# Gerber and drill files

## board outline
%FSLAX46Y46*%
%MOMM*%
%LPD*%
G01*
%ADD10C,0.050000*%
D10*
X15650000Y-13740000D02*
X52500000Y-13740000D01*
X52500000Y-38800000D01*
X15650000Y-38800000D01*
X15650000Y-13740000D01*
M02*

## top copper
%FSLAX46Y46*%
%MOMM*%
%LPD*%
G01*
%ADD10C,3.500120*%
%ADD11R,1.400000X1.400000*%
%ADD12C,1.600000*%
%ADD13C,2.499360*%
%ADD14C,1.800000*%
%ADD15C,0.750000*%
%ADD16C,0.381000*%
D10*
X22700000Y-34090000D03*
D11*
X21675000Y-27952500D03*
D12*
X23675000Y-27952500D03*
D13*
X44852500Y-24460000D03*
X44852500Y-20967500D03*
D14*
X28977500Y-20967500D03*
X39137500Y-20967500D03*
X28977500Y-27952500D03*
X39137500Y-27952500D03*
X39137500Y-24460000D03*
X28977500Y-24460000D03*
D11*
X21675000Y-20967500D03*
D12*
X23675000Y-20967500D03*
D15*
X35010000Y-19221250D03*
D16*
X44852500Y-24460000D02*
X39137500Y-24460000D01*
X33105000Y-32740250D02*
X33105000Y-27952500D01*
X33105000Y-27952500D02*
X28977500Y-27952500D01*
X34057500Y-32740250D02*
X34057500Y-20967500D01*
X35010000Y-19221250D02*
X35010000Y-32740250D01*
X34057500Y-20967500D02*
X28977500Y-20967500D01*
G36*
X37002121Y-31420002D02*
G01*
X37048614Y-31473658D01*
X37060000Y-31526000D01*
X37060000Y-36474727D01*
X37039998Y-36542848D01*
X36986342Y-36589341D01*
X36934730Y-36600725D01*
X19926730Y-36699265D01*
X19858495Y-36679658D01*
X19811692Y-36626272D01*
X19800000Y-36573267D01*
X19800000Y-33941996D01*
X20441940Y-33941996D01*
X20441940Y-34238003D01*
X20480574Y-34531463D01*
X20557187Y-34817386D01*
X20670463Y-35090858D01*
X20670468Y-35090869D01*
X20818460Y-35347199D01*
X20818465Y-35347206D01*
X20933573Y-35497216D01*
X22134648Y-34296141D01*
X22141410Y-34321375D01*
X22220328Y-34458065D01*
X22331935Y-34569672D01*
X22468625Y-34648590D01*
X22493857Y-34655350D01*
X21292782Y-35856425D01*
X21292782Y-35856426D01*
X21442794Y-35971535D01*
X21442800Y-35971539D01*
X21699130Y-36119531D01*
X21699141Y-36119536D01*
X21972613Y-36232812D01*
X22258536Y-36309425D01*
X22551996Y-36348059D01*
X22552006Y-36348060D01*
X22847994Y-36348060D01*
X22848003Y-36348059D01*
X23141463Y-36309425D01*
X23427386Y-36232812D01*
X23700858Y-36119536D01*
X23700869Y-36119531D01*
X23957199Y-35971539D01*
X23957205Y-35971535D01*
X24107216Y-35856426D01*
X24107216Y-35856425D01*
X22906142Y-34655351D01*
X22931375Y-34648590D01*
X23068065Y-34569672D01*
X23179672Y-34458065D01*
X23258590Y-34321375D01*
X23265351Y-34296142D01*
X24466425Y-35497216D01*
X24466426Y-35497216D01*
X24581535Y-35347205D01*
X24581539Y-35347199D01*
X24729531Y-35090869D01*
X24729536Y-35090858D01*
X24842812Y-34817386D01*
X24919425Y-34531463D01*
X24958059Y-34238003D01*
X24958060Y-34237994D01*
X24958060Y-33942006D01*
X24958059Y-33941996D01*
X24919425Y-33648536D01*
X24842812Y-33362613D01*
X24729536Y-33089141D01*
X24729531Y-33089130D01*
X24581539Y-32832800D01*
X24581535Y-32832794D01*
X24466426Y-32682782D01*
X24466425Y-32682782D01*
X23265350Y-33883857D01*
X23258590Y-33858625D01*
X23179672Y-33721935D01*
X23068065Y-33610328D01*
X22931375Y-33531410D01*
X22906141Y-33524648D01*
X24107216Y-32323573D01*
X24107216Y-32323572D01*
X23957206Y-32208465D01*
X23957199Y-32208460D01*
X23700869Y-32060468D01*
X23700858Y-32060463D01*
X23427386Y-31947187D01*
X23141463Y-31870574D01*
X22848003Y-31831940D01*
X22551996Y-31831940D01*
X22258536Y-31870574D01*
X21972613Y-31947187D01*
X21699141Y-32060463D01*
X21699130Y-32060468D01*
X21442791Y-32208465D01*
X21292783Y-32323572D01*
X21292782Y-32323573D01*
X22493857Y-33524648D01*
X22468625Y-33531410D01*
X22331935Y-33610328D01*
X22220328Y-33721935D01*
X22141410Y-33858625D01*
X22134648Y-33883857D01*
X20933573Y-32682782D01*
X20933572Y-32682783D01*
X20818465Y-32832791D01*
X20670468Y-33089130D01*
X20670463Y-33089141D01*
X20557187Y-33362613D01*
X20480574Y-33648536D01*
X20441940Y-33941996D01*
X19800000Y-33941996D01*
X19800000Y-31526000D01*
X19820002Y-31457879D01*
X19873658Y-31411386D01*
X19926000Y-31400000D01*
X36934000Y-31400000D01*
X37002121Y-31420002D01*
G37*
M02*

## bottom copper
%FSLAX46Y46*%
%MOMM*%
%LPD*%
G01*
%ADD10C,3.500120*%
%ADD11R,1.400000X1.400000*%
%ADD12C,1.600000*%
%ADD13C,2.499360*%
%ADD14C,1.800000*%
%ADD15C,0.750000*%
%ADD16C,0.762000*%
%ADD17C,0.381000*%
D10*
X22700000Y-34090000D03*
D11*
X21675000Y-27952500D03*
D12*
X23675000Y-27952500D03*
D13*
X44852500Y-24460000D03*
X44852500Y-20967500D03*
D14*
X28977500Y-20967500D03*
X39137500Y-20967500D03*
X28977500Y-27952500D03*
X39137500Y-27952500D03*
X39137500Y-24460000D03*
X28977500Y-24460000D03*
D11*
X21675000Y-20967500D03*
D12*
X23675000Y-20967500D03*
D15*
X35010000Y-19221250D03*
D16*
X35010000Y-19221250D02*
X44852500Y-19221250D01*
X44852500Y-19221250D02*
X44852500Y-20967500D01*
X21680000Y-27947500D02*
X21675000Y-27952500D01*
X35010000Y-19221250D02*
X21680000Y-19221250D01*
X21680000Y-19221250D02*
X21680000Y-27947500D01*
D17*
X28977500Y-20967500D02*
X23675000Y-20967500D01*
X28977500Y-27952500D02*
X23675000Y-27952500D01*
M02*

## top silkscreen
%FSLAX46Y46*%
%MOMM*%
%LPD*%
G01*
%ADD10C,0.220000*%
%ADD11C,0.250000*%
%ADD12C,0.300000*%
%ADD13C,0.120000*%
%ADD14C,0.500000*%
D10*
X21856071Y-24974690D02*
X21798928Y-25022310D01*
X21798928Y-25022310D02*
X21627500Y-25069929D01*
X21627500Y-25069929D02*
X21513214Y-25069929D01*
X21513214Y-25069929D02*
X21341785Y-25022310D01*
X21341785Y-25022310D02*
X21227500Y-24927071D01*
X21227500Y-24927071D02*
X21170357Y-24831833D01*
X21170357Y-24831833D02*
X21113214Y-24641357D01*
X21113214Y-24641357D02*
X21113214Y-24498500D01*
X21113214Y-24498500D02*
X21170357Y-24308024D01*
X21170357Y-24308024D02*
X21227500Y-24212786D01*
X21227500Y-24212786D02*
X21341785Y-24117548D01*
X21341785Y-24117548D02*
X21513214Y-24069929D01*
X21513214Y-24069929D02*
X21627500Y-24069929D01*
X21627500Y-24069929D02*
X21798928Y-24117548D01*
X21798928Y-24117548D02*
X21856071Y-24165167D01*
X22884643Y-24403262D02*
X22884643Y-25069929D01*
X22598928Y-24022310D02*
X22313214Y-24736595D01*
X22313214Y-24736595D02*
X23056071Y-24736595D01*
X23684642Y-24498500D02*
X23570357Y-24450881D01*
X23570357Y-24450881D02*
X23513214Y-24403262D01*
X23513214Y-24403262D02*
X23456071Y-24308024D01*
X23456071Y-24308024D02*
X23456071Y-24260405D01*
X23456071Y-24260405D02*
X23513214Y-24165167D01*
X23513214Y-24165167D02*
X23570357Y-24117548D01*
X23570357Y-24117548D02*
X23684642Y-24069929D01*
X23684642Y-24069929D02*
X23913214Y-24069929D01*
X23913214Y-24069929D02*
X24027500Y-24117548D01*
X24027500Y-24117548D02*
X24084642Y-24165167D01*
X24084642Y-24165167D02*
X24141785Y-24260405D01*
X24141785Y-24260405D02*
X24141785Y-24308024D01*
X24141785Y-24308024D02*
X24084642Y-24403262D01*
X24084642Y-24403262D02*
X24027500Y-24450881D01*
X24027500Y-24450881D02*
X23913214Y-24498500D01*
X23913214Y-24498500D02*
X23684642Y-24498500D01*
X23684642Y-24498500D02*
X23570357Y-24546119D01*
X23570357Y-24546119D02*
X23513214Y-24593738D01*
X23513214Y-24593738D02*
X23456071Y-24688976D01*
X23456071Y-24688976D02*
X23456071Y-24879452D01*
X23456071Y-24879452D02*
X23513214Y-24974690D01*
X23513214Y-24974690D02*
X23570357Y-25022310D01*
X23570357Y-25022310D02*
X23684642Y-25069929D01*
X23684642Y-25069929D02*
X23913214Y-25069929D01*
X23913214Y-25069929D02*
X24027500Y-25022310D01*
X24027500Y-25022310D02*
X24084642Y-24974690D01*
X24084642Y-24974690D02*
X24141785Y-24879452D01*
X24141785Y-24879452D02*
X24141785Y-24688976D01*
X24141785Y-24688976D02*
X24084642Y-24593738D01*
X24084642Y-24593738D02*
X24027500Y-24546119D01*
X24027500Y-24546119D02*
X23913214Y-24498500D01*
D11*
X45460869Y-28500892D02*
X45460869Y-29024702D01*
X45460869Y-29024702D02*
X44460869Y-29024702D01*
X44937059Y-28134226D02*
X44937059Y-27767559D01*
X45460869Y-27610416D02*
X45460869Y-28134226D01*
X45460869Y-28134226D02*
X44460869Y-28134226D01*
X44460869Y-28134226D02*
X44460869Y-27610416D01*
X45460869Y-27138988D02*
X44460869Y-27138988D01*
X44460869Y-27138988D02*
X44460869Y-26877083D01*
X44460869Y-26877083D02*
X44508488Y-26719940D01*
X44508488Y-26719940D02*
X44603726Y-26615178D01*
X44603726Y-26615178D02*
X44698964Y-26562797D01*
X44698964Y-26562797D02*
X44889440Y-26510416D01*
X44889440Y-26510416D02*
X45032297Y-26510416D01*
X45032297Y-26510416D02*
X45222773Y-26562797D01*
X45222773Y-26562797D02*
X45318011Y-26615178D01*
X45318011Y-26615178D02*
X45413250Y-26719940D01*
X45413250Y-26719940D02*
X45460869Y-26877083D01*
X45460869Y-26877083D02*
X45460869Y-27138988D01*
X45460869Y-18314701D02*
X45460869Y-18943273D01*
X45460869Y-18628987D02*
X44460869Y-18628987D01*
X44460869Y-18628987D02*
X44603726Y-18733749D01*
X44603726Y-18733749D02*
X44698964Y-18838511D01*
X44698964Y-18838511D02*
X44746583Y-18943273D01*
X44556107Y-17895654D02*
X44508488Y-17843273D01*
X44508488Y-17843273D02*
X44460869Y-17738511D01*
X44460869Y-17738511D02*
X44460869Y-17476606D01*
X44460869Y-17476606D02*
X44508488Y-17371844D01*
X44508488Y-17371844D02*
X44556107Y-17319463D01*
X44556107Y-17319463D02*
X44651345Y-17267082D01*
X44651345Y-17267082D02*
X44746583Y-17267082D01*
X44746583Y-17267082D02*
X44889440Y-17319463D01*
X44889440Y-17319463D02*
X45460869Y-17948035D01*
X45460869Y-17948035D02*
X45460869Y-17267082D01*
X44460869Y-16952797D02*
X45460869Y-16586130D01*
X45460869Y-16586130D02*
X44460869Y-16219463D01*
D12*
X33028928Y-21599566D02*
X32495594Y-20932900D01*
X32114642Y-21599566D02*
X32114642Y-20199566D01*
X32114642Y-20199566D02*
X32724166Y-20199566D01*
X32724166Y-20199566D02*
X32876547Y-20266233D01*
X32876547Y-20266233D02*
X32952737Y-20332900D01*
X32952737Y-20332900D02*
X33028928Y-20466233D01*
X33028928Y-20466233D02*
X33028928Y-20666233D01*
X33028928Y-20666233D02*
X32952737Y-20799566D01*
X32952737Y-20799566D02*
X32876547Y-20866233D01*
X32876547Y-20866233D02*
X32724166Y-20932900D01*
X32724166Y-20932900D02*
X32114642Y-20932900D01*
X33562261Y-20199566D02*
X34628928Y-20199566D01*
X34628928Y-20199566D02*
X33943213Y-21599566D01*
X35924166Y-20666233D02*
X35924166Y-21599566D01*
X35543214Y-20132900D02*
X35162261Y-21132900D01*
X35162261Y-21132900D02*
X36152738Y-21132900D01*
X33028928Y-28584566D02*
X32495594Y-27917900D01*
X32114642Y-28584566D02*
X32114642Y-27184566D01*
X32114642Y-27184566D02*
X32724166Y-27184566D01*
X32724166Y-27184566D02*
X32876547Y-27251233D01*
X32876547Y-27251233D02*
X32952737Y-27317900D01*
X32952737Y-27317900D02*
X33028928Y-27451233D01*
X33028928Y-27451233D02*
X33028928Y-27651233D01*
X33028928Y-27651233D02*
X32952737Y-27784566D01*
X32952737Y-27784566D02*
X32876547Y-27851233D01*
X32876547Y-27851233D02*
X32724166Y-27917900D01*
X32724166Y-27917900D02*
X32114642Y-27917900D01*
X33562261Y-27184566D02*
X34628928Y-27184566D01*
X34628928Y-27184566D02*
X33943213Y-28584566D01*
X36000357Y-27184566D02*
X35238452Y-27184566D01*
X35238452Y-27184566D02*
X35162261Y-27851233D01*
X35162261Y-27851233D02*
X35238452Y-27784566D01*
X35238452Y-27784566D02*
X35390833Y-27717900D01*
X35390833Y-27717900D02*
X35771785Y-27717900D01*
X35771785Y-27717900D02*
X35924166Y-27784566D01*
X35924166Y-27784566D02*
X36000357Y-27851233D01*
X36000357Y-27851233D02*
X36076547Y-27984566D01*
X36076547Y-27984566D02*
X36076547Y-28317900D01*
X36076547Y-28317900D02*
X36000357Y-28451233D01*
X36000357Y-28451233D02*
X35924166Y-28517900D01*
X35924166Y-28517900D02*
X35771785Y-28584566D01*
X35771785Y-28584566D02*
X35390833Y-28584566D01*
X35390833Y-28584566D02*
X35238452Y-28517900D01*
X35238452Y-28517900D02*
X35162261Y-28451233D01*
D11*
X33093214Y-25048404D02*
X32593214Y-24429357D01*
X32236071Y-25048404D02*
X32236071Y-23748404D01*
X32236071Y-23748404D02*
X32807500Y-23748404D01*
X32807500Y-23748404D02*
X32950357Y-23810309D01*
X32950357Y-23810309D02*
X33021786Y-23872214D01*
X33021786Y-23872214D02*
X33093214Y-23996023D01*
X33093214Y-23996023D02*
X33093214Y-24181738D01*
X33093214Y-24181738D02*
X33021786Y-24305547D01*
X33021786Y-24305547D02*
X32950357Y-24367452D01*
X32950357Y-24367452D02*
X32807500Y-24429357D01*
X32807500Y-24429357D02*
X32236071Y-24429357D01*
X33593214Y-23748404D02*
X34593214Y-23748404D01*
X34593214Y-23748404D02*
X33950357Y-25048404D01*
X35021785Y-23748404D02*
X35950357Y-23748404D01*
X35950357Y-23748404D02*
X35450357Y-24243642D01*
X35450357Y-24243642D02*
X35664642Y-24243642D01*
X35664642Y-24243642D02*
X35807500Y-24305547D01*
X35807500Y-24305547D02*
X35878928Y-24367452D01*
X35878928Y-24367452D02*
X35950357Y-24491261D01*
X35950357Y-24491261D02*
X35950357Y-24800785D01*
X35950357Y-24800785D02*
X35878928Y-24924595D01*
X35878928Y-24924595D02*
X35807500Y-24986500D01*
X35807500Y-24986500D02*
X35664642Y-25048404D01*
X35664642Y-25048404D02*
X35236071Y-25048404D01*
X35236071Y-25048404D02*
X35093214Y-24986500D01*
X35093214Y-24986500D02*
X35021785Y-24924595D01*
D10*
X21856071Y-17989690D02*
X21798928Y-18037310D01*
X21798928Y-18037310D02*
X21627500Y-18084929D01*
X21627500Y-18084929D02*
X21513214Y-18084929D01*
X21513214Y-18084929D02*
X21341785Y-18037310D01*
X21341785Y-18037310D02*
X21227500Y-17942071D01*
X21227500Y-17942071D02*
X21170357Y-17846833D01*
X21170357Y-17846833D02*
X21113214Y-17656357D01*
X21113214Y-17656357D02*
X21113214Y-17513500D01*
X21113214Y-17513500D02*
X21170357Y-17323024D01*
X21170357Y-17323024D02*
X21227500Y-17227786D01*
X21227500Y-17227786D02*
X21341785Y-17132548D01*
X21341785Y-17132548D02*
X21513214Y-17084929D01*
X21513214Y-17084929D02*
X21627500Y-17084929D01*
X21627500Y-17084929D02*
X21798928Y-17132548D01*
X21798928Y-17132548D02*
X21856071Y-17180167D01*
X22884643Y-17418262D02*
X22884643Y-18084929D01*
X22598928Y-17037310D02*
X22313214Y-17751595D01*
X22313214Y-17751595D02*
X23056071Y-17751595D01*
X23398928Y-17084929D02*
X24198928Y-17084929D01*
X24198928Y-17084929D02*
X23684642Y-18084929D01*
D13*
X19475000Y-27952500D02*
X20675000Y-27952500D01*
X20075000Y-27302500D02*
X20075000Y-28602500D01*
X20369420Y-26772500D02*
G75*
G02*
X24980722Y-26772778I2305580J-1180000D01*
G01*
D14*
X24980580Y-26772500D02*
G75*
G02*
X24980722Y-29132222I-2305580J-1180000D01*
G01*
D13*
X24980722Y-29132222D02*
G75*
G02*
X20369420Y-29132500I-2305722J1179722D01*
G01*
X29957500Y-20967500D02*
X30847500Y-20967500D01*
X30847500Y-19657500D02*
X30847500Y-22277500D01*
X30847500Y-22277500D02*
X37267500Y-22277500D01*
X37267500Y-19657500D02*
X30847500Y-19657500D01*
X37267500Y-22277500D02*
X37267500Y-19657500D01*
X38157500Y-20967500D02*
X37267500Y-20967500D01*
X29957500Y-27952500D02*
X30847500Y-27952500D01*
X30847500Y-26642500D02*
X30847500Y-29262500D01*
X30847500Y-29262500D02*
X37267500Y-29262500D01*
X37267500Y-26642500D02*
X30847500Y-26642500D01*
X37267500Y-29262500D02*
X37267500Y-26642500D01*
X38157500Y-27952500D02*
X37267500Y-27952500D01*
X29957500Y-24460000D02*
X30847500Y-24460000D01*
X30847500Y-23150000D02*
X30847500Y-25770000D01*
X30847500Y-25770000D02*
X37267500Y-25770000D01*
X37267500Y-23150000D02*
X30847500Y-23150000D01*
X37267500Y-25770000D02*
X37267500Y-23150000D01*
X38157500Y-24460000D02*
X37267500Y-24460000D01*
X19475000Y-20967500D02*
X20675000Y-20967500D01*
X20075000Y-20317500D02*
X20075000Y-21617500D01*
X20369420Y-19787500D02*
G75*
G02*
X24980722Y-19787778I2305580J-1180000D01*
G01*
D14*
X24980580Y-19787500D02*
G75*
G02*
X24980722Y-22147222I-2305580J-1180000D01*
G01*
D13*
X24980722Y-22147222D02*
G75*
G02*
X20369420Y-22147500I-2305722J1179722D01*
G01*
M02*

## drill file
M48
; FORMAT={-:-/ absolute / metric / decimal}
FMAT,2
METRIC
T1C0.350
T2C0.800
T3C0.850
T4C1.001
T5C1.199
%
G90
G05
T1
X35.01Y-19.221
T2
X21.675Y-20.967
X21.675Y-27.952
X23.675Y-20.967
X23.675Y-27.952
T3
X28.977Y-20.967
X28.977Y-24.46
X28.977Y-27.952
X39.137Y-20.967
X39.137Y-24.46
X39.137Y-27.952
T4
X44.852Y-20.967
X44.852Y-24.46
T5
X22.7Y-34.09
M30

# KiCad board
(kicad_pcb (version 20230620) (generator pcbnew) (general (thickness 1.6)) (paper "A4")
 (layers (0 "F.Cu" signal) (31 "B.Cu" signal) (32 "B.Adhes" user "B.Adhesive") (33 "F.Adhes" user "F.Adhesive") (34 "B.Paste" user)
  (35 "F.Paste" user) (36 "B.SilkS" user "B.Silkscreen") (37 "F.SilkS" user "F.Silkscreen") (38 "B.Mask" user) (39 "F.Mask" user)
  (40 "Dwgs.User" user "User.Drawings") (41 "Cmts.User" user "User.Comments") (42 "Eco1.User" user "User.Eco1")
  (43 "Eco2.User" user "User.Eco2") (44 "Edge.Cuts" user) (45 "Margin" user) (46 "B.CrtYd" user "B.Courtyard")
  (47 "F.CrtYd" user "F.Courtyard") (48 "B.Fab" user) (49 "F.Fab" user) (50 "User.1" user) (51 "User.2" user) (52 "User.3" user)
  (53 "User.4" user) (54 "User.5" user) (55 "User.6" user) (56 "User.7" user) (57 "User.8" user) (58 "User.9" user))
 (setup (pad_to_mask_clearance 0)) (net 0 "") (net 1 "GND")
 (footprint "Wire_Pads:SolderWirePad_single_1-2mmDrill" (layer "F.Cu") (at 22.7 34.09)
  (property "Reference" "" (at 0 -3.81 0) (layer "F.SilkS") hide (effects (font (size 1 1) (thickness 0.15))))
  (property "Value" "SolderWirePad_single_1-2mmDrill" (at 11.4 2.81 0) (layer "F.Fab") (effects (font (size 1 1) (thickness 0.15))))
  (pad "1" thru_hole circle (at 0 0) (size 3.50012 3.50012) (drill 1.19888) (layers "*.Cu" "*.Mask") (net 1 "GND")))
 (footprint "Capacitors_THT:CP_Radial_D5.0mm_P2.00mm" (layer "F.Cu") (at 21.675 27.9525)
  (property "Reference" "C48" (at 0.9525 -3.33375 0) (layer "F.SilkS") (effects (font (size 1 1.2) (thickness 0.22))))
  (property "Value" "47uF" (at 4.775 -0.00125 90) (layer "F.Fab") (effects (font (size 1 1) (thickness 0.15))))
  (fp_line (start -2.2 0) (end -1 0) (stroke (width 0.12) (type solid)) (layer "F.SilkS"))
  (fp_line (start -1.6 -0.65) (end -1.6 0.65) (stroke (width 0.12) (type solid)) (layer "F.SilkS"))
  (fp_arc (start -1.30558 -1.18) (mid 1.000156 -2.59) (end 3.305722 -1.179722) (stroke (width 0.12) (type solid)) (layer "F.SilkS"))
  (fp_arc (start 3.30558 -1.18) (mid 3.59 -0.000156) (end 3.305722 1.179722) (stroke (width 0.5) (type solid)) (layer "F.SilkS"))
  (fp_arc (start 3.305722 1.179722) (mid 1.000156 2.59) (end -1.30558 1.18) (stroke (width 0.12) (type solid)) (layer "F.SilkS"))
  (pad "1" thru_hole rect (at 0 0) (size 1.4 1.4) (drill 0.8) (layers "*.Cu" "*.Mask") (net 1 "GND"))
  (pad "2" thru_hole circle (at 2 0) (size 1.6 1.6) (drill 0.8) (layers "*.Cu" "*.Mask") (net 1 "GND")))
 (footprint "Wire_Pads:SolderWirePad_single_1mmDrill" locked (layer "F.Cu") (at 44.8525 24.46)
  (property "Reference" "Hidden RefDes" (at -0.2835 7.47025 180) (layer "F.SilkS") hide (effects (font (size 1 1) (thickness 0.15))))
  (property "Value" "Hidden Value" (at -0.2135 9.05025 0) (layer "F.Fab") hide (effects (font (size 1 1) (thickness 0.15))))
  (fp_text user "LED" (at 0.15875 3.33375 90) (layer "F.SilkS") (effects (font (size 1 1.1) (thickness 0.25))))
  (pad "1" thru_hole circle locked (at 0 0) (size 2.49936 2.49936) (drill 1.00076) (layers "*.Cu" "*.Mask")))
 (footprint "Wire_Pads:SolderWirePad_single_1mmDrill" (layer "F.Cu") (at 44.8525 20.9675)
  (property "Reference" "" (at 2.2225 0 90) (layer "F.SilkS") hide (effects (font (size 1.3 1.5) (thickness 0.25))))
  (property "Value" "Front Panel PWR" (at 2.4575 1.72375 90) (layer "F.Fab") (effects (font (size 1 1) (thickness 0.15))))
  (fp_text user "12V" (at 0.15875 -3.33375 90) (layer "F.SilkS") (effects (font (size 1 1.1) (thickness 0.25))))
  (pad "1" thru_hole circle (at 0 0) (size 2.49936 2.49936) (drill 1.00076) (layers "*.Cu" "*.Mask") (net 1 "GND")))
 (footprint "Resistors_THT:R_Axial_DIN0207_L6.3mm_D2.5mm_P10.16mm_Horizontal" (layer "F.Cu") (at 28.9775 20.9675)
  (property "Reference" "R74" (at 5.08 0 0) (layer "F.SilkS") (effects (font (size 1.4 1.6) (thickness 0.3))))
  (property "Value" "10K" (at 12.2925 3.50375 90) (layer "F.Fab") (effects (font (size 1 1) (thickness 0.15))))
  (fp_line (start 0.98 0) (end 1.87 0) (stroke (width 0.12) (type solid)) (layer "F.SilkS"))
  (fp_line (start 1.87 -1.31) (end 1.87 1.31) (stroke (width 0.12) (type solid)) (layer "F.SilkS"))
  (fp_line (start 1.87 1.31) (end 8.29 1.31) (stroke (width 0.12) (type solid)) (layer "F.SilkS"))
  (fp_line (start 8.29 -1.31) (end 1.87 -1.31) (stroke (width 0.12) (type solid)) (layer "F.SilkS"))
  (fp_line (start 8.29 1.31) (end 8.29 -1.31) (stroke (width 0.12) (type solid)) (layer "F.SilkS"))
  (fp_line (start 9.18 0) (end 8.29 0) (stroke (width 0.12) (type solid)) (layer "F.SilkS"))
  (pad "1" thru_hole circle (at 0 0) (size 1.8 1.8) (drill 0.85) (layers "*.Cu" "*.Mask") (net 1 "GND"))
  (pad "2" thru_hole circle (at 10.16 0) (size 1.8 1.8) (drill 0.85) (layers "*.Cu" "*.Mask")))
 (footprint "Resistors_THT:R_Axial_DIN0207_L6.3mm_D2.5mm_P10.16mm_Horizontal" (layer "F.Cu") (at 28.9775 27.9525)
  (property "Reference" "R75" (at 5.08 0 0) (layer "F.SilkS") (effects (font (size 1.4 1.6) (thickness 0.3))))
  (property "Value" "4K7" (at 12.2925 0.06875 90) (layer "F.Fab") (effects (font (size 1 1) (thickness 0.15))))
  (fp_line (start 0.98 0) (end 1.87 0) (stroke (width 0.12) (type solid)) (layer "F.SilkS"))
  (fp_line (start 1.87 -1.31) (end 1.87 1.31) (stroke (width 0.12) (type solid)) (layer "F.SilkS"))
  (fp_line (start 1.87 1.31) (end 8.29 1.31) (stroke (width 0.12) (type solid)) (layer "F.SilkS"))
  (fp_line (start 8.29 -1.31) (end 1.87 -1.31) (stroke (width 0.12) (type solid)) (layer "F.SilkS"))
  (fp_line (start 8.29 1.31) (end 8.29 -1.31) (stroke (width 0.12) (type solid)) (layer "F.SilkS"))
  (fp_line (start 9.18 0) (end 8.29 0) (stroke (width 0.12) (type solid)) (layer "F.SilkS"))
  (pad "1" thru_hole circle (at 0 0) (size 1.8 1.8) (drill 0.85) (layers "*.Cu" "*.Mask") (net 1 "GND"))
  (pad "2" thru_hole circle (at 10.16 0) (size 1.8 1.8) (drill 0.85) (layers "*.Cu" "*.Mask")))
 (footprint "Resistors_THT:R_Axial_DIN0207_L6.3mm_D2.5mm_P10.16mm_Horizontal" (layer "F.Cu") (at 39.1375 24.46 180)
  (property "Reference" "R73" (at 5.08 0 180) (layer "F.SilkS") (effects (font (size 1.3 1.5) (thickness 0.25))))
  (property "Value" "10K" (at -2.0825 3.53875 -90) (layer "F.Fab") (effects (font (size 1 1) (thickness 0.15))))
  (fp_line (start 9.18 0) (end 8.29 0) (stroke (width 0.12) (type solid)) (layer "F.SilkS"))
  (fp_line (start 8.29 1.31) (end 8.29 -1.31) (stroke (width 0.12) (type solid)) (layer "F.SilkS"))
  (fp_line (start 8.29 -1.31) (end 1.87 -1.31) (stroke (width 0.12) (type solid)) (layer "F.SilkS"))
  (fp_line (start 1.87 1.31) (end 8.29 1.31) (stroke (width 0.12) (type solid)) (layer "F.SilkS"))
  (fp_line (start 1.87 -1.31) (end 1.87 1.31) (stroke (width 0.12) (type solid)) (layer "F.SilkS"))
  (fp_line (start 0.98 0) (end 1.87 0) (stroke (width 0.12) (type solid)) (layer "F.SilkS"))
  (pad "1" thru_hole circle (at 0 0 180) (size 1.8 1.8) (drill 0.85) (layers "*.Cu" "*.Mask"))
  (pad "2" thru_hole circle (at 10.16 0 180) (size 1.8 1.8) (drill 0.85) (layers "*.Cu" "*.Mask")))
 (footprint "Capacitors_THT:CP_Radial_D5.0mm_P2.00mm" (layer "F.Cu") (at 21.675 20.9675)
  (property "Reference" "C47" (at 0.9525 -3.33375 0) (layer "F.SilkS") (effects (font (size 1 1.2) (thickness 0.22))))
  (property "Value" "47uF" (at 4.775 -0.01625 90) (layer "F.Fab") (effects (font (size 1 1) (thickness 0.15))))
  (fp_line (start -2.2 0) (end -1 0) (stroke (width 0.12) (type solid)) (layer "F.SilkS"))
  (fp_line (start -1.6 -0.65) (end -1.6 0.65) (stroke (width 0.12) (type solid)) (layer "F.SilkS"))
  (fp_arc (start -1.30558 -1.18) (mid 1.000156 -2.59) (end 3.305722 -1.179722) (stroke (width 0.12) (type solid)) (layer "F.SilkS"))
  (fp_arc (start 3.30558 -1.18) (mid 3.59 -0.000156) (end 3.305722 1.179722) (stroke (width 0.5) (type solid)) (layer "F.SilkS"))
  (fp_arc (start 3.305722 1.179722) (mid 1.000156 2.59) (end -1.30558 1.18) (stroke (width 0.12) (type solid)) (layer "F.SilkS"))
  (pad "1" thru_hole rect (at 0 0) (size 1.4 1.4) (drill 0.8) (layers "*.Cu" "*.Mask") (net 1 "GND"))
  (pad "2" thru_hole circle (at 2 0) (size 1.6 1.6) (drill 0.8) (layers "*.Cu" "*.Mask") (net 1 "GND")))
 (gr_rect (start 15.65 13.74) (end 52.5 38.8) (stroke (width 0.05) (type solid)) (fill none) (layer "Edge.Cuts"))
 (segment (start 44.8525 24.46) (end 39.1375 24.46) (width 0.381) (layer "F.Cu") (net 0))
 (segment (start 33.105 32.74025) (end 33.105 27.9525) (width 0.381) (layer "F.Cu") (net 1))
 (segment (start 33.105 27.9525) (end 28.9775 27.9525) (width 0.381) (layer "F.Cu") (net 1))
 (segment (start 34.0575 32.74025) (end 34.0575 20.9675) (width 0.381) (layer "F.Cu") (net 1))
 (segment (start 35.01 19.22125) (end 35.01 32.74025) (width 0.381) (layer "F.Cu") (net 1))
 (segment (start 34.0575 20.9675) (end 28.9775 20.9675) (width 0.381) (layer "F.Cu") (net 1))
 (via (at 35.01 19.22125) (size 0.75) (drill 0.35) (layers "F.Cu" "B.Cu") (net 1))
 (segment (start 35.01 19.22125) (end 44.8525 19.22125) (width 0.762) (layer "B.Cu") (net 1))
 (segment (start 44.8525 19.22125) (end 44.8525 20.9675) (width 0.762) (layer "B.Cu") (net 1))
 (segment (start 21.68 27.9475) (end 21.675 27.9525) (width 0.762) (layer "B.Cu") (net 1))
 (segment (start 35.01 19.22125) (end 21.68 19.22125) (width 0.762) (layer "B.Cu") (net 1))
 (segment (start 21.68 19.22125) (end 21.68 27.9475) (width 0.762) (layer "B.Cu") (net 1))
 (segment (start 28.9775 20.9675) (end 23.675 20.9675) (width 0.381) (layer "B.Cu") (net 1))
 (segment (start 28.9775 27.9525) (end 23.675 27.9525) (width 0.381) (layer "B.Cu") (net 1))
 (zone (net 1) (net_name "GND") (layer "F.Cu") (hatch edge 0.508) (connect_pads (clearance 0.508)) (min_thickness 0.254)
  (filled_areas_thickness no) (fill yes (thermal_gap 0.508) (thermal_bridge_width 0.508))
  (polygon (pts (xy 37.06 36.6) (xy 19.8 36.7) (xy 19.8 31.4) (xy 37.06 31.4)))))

